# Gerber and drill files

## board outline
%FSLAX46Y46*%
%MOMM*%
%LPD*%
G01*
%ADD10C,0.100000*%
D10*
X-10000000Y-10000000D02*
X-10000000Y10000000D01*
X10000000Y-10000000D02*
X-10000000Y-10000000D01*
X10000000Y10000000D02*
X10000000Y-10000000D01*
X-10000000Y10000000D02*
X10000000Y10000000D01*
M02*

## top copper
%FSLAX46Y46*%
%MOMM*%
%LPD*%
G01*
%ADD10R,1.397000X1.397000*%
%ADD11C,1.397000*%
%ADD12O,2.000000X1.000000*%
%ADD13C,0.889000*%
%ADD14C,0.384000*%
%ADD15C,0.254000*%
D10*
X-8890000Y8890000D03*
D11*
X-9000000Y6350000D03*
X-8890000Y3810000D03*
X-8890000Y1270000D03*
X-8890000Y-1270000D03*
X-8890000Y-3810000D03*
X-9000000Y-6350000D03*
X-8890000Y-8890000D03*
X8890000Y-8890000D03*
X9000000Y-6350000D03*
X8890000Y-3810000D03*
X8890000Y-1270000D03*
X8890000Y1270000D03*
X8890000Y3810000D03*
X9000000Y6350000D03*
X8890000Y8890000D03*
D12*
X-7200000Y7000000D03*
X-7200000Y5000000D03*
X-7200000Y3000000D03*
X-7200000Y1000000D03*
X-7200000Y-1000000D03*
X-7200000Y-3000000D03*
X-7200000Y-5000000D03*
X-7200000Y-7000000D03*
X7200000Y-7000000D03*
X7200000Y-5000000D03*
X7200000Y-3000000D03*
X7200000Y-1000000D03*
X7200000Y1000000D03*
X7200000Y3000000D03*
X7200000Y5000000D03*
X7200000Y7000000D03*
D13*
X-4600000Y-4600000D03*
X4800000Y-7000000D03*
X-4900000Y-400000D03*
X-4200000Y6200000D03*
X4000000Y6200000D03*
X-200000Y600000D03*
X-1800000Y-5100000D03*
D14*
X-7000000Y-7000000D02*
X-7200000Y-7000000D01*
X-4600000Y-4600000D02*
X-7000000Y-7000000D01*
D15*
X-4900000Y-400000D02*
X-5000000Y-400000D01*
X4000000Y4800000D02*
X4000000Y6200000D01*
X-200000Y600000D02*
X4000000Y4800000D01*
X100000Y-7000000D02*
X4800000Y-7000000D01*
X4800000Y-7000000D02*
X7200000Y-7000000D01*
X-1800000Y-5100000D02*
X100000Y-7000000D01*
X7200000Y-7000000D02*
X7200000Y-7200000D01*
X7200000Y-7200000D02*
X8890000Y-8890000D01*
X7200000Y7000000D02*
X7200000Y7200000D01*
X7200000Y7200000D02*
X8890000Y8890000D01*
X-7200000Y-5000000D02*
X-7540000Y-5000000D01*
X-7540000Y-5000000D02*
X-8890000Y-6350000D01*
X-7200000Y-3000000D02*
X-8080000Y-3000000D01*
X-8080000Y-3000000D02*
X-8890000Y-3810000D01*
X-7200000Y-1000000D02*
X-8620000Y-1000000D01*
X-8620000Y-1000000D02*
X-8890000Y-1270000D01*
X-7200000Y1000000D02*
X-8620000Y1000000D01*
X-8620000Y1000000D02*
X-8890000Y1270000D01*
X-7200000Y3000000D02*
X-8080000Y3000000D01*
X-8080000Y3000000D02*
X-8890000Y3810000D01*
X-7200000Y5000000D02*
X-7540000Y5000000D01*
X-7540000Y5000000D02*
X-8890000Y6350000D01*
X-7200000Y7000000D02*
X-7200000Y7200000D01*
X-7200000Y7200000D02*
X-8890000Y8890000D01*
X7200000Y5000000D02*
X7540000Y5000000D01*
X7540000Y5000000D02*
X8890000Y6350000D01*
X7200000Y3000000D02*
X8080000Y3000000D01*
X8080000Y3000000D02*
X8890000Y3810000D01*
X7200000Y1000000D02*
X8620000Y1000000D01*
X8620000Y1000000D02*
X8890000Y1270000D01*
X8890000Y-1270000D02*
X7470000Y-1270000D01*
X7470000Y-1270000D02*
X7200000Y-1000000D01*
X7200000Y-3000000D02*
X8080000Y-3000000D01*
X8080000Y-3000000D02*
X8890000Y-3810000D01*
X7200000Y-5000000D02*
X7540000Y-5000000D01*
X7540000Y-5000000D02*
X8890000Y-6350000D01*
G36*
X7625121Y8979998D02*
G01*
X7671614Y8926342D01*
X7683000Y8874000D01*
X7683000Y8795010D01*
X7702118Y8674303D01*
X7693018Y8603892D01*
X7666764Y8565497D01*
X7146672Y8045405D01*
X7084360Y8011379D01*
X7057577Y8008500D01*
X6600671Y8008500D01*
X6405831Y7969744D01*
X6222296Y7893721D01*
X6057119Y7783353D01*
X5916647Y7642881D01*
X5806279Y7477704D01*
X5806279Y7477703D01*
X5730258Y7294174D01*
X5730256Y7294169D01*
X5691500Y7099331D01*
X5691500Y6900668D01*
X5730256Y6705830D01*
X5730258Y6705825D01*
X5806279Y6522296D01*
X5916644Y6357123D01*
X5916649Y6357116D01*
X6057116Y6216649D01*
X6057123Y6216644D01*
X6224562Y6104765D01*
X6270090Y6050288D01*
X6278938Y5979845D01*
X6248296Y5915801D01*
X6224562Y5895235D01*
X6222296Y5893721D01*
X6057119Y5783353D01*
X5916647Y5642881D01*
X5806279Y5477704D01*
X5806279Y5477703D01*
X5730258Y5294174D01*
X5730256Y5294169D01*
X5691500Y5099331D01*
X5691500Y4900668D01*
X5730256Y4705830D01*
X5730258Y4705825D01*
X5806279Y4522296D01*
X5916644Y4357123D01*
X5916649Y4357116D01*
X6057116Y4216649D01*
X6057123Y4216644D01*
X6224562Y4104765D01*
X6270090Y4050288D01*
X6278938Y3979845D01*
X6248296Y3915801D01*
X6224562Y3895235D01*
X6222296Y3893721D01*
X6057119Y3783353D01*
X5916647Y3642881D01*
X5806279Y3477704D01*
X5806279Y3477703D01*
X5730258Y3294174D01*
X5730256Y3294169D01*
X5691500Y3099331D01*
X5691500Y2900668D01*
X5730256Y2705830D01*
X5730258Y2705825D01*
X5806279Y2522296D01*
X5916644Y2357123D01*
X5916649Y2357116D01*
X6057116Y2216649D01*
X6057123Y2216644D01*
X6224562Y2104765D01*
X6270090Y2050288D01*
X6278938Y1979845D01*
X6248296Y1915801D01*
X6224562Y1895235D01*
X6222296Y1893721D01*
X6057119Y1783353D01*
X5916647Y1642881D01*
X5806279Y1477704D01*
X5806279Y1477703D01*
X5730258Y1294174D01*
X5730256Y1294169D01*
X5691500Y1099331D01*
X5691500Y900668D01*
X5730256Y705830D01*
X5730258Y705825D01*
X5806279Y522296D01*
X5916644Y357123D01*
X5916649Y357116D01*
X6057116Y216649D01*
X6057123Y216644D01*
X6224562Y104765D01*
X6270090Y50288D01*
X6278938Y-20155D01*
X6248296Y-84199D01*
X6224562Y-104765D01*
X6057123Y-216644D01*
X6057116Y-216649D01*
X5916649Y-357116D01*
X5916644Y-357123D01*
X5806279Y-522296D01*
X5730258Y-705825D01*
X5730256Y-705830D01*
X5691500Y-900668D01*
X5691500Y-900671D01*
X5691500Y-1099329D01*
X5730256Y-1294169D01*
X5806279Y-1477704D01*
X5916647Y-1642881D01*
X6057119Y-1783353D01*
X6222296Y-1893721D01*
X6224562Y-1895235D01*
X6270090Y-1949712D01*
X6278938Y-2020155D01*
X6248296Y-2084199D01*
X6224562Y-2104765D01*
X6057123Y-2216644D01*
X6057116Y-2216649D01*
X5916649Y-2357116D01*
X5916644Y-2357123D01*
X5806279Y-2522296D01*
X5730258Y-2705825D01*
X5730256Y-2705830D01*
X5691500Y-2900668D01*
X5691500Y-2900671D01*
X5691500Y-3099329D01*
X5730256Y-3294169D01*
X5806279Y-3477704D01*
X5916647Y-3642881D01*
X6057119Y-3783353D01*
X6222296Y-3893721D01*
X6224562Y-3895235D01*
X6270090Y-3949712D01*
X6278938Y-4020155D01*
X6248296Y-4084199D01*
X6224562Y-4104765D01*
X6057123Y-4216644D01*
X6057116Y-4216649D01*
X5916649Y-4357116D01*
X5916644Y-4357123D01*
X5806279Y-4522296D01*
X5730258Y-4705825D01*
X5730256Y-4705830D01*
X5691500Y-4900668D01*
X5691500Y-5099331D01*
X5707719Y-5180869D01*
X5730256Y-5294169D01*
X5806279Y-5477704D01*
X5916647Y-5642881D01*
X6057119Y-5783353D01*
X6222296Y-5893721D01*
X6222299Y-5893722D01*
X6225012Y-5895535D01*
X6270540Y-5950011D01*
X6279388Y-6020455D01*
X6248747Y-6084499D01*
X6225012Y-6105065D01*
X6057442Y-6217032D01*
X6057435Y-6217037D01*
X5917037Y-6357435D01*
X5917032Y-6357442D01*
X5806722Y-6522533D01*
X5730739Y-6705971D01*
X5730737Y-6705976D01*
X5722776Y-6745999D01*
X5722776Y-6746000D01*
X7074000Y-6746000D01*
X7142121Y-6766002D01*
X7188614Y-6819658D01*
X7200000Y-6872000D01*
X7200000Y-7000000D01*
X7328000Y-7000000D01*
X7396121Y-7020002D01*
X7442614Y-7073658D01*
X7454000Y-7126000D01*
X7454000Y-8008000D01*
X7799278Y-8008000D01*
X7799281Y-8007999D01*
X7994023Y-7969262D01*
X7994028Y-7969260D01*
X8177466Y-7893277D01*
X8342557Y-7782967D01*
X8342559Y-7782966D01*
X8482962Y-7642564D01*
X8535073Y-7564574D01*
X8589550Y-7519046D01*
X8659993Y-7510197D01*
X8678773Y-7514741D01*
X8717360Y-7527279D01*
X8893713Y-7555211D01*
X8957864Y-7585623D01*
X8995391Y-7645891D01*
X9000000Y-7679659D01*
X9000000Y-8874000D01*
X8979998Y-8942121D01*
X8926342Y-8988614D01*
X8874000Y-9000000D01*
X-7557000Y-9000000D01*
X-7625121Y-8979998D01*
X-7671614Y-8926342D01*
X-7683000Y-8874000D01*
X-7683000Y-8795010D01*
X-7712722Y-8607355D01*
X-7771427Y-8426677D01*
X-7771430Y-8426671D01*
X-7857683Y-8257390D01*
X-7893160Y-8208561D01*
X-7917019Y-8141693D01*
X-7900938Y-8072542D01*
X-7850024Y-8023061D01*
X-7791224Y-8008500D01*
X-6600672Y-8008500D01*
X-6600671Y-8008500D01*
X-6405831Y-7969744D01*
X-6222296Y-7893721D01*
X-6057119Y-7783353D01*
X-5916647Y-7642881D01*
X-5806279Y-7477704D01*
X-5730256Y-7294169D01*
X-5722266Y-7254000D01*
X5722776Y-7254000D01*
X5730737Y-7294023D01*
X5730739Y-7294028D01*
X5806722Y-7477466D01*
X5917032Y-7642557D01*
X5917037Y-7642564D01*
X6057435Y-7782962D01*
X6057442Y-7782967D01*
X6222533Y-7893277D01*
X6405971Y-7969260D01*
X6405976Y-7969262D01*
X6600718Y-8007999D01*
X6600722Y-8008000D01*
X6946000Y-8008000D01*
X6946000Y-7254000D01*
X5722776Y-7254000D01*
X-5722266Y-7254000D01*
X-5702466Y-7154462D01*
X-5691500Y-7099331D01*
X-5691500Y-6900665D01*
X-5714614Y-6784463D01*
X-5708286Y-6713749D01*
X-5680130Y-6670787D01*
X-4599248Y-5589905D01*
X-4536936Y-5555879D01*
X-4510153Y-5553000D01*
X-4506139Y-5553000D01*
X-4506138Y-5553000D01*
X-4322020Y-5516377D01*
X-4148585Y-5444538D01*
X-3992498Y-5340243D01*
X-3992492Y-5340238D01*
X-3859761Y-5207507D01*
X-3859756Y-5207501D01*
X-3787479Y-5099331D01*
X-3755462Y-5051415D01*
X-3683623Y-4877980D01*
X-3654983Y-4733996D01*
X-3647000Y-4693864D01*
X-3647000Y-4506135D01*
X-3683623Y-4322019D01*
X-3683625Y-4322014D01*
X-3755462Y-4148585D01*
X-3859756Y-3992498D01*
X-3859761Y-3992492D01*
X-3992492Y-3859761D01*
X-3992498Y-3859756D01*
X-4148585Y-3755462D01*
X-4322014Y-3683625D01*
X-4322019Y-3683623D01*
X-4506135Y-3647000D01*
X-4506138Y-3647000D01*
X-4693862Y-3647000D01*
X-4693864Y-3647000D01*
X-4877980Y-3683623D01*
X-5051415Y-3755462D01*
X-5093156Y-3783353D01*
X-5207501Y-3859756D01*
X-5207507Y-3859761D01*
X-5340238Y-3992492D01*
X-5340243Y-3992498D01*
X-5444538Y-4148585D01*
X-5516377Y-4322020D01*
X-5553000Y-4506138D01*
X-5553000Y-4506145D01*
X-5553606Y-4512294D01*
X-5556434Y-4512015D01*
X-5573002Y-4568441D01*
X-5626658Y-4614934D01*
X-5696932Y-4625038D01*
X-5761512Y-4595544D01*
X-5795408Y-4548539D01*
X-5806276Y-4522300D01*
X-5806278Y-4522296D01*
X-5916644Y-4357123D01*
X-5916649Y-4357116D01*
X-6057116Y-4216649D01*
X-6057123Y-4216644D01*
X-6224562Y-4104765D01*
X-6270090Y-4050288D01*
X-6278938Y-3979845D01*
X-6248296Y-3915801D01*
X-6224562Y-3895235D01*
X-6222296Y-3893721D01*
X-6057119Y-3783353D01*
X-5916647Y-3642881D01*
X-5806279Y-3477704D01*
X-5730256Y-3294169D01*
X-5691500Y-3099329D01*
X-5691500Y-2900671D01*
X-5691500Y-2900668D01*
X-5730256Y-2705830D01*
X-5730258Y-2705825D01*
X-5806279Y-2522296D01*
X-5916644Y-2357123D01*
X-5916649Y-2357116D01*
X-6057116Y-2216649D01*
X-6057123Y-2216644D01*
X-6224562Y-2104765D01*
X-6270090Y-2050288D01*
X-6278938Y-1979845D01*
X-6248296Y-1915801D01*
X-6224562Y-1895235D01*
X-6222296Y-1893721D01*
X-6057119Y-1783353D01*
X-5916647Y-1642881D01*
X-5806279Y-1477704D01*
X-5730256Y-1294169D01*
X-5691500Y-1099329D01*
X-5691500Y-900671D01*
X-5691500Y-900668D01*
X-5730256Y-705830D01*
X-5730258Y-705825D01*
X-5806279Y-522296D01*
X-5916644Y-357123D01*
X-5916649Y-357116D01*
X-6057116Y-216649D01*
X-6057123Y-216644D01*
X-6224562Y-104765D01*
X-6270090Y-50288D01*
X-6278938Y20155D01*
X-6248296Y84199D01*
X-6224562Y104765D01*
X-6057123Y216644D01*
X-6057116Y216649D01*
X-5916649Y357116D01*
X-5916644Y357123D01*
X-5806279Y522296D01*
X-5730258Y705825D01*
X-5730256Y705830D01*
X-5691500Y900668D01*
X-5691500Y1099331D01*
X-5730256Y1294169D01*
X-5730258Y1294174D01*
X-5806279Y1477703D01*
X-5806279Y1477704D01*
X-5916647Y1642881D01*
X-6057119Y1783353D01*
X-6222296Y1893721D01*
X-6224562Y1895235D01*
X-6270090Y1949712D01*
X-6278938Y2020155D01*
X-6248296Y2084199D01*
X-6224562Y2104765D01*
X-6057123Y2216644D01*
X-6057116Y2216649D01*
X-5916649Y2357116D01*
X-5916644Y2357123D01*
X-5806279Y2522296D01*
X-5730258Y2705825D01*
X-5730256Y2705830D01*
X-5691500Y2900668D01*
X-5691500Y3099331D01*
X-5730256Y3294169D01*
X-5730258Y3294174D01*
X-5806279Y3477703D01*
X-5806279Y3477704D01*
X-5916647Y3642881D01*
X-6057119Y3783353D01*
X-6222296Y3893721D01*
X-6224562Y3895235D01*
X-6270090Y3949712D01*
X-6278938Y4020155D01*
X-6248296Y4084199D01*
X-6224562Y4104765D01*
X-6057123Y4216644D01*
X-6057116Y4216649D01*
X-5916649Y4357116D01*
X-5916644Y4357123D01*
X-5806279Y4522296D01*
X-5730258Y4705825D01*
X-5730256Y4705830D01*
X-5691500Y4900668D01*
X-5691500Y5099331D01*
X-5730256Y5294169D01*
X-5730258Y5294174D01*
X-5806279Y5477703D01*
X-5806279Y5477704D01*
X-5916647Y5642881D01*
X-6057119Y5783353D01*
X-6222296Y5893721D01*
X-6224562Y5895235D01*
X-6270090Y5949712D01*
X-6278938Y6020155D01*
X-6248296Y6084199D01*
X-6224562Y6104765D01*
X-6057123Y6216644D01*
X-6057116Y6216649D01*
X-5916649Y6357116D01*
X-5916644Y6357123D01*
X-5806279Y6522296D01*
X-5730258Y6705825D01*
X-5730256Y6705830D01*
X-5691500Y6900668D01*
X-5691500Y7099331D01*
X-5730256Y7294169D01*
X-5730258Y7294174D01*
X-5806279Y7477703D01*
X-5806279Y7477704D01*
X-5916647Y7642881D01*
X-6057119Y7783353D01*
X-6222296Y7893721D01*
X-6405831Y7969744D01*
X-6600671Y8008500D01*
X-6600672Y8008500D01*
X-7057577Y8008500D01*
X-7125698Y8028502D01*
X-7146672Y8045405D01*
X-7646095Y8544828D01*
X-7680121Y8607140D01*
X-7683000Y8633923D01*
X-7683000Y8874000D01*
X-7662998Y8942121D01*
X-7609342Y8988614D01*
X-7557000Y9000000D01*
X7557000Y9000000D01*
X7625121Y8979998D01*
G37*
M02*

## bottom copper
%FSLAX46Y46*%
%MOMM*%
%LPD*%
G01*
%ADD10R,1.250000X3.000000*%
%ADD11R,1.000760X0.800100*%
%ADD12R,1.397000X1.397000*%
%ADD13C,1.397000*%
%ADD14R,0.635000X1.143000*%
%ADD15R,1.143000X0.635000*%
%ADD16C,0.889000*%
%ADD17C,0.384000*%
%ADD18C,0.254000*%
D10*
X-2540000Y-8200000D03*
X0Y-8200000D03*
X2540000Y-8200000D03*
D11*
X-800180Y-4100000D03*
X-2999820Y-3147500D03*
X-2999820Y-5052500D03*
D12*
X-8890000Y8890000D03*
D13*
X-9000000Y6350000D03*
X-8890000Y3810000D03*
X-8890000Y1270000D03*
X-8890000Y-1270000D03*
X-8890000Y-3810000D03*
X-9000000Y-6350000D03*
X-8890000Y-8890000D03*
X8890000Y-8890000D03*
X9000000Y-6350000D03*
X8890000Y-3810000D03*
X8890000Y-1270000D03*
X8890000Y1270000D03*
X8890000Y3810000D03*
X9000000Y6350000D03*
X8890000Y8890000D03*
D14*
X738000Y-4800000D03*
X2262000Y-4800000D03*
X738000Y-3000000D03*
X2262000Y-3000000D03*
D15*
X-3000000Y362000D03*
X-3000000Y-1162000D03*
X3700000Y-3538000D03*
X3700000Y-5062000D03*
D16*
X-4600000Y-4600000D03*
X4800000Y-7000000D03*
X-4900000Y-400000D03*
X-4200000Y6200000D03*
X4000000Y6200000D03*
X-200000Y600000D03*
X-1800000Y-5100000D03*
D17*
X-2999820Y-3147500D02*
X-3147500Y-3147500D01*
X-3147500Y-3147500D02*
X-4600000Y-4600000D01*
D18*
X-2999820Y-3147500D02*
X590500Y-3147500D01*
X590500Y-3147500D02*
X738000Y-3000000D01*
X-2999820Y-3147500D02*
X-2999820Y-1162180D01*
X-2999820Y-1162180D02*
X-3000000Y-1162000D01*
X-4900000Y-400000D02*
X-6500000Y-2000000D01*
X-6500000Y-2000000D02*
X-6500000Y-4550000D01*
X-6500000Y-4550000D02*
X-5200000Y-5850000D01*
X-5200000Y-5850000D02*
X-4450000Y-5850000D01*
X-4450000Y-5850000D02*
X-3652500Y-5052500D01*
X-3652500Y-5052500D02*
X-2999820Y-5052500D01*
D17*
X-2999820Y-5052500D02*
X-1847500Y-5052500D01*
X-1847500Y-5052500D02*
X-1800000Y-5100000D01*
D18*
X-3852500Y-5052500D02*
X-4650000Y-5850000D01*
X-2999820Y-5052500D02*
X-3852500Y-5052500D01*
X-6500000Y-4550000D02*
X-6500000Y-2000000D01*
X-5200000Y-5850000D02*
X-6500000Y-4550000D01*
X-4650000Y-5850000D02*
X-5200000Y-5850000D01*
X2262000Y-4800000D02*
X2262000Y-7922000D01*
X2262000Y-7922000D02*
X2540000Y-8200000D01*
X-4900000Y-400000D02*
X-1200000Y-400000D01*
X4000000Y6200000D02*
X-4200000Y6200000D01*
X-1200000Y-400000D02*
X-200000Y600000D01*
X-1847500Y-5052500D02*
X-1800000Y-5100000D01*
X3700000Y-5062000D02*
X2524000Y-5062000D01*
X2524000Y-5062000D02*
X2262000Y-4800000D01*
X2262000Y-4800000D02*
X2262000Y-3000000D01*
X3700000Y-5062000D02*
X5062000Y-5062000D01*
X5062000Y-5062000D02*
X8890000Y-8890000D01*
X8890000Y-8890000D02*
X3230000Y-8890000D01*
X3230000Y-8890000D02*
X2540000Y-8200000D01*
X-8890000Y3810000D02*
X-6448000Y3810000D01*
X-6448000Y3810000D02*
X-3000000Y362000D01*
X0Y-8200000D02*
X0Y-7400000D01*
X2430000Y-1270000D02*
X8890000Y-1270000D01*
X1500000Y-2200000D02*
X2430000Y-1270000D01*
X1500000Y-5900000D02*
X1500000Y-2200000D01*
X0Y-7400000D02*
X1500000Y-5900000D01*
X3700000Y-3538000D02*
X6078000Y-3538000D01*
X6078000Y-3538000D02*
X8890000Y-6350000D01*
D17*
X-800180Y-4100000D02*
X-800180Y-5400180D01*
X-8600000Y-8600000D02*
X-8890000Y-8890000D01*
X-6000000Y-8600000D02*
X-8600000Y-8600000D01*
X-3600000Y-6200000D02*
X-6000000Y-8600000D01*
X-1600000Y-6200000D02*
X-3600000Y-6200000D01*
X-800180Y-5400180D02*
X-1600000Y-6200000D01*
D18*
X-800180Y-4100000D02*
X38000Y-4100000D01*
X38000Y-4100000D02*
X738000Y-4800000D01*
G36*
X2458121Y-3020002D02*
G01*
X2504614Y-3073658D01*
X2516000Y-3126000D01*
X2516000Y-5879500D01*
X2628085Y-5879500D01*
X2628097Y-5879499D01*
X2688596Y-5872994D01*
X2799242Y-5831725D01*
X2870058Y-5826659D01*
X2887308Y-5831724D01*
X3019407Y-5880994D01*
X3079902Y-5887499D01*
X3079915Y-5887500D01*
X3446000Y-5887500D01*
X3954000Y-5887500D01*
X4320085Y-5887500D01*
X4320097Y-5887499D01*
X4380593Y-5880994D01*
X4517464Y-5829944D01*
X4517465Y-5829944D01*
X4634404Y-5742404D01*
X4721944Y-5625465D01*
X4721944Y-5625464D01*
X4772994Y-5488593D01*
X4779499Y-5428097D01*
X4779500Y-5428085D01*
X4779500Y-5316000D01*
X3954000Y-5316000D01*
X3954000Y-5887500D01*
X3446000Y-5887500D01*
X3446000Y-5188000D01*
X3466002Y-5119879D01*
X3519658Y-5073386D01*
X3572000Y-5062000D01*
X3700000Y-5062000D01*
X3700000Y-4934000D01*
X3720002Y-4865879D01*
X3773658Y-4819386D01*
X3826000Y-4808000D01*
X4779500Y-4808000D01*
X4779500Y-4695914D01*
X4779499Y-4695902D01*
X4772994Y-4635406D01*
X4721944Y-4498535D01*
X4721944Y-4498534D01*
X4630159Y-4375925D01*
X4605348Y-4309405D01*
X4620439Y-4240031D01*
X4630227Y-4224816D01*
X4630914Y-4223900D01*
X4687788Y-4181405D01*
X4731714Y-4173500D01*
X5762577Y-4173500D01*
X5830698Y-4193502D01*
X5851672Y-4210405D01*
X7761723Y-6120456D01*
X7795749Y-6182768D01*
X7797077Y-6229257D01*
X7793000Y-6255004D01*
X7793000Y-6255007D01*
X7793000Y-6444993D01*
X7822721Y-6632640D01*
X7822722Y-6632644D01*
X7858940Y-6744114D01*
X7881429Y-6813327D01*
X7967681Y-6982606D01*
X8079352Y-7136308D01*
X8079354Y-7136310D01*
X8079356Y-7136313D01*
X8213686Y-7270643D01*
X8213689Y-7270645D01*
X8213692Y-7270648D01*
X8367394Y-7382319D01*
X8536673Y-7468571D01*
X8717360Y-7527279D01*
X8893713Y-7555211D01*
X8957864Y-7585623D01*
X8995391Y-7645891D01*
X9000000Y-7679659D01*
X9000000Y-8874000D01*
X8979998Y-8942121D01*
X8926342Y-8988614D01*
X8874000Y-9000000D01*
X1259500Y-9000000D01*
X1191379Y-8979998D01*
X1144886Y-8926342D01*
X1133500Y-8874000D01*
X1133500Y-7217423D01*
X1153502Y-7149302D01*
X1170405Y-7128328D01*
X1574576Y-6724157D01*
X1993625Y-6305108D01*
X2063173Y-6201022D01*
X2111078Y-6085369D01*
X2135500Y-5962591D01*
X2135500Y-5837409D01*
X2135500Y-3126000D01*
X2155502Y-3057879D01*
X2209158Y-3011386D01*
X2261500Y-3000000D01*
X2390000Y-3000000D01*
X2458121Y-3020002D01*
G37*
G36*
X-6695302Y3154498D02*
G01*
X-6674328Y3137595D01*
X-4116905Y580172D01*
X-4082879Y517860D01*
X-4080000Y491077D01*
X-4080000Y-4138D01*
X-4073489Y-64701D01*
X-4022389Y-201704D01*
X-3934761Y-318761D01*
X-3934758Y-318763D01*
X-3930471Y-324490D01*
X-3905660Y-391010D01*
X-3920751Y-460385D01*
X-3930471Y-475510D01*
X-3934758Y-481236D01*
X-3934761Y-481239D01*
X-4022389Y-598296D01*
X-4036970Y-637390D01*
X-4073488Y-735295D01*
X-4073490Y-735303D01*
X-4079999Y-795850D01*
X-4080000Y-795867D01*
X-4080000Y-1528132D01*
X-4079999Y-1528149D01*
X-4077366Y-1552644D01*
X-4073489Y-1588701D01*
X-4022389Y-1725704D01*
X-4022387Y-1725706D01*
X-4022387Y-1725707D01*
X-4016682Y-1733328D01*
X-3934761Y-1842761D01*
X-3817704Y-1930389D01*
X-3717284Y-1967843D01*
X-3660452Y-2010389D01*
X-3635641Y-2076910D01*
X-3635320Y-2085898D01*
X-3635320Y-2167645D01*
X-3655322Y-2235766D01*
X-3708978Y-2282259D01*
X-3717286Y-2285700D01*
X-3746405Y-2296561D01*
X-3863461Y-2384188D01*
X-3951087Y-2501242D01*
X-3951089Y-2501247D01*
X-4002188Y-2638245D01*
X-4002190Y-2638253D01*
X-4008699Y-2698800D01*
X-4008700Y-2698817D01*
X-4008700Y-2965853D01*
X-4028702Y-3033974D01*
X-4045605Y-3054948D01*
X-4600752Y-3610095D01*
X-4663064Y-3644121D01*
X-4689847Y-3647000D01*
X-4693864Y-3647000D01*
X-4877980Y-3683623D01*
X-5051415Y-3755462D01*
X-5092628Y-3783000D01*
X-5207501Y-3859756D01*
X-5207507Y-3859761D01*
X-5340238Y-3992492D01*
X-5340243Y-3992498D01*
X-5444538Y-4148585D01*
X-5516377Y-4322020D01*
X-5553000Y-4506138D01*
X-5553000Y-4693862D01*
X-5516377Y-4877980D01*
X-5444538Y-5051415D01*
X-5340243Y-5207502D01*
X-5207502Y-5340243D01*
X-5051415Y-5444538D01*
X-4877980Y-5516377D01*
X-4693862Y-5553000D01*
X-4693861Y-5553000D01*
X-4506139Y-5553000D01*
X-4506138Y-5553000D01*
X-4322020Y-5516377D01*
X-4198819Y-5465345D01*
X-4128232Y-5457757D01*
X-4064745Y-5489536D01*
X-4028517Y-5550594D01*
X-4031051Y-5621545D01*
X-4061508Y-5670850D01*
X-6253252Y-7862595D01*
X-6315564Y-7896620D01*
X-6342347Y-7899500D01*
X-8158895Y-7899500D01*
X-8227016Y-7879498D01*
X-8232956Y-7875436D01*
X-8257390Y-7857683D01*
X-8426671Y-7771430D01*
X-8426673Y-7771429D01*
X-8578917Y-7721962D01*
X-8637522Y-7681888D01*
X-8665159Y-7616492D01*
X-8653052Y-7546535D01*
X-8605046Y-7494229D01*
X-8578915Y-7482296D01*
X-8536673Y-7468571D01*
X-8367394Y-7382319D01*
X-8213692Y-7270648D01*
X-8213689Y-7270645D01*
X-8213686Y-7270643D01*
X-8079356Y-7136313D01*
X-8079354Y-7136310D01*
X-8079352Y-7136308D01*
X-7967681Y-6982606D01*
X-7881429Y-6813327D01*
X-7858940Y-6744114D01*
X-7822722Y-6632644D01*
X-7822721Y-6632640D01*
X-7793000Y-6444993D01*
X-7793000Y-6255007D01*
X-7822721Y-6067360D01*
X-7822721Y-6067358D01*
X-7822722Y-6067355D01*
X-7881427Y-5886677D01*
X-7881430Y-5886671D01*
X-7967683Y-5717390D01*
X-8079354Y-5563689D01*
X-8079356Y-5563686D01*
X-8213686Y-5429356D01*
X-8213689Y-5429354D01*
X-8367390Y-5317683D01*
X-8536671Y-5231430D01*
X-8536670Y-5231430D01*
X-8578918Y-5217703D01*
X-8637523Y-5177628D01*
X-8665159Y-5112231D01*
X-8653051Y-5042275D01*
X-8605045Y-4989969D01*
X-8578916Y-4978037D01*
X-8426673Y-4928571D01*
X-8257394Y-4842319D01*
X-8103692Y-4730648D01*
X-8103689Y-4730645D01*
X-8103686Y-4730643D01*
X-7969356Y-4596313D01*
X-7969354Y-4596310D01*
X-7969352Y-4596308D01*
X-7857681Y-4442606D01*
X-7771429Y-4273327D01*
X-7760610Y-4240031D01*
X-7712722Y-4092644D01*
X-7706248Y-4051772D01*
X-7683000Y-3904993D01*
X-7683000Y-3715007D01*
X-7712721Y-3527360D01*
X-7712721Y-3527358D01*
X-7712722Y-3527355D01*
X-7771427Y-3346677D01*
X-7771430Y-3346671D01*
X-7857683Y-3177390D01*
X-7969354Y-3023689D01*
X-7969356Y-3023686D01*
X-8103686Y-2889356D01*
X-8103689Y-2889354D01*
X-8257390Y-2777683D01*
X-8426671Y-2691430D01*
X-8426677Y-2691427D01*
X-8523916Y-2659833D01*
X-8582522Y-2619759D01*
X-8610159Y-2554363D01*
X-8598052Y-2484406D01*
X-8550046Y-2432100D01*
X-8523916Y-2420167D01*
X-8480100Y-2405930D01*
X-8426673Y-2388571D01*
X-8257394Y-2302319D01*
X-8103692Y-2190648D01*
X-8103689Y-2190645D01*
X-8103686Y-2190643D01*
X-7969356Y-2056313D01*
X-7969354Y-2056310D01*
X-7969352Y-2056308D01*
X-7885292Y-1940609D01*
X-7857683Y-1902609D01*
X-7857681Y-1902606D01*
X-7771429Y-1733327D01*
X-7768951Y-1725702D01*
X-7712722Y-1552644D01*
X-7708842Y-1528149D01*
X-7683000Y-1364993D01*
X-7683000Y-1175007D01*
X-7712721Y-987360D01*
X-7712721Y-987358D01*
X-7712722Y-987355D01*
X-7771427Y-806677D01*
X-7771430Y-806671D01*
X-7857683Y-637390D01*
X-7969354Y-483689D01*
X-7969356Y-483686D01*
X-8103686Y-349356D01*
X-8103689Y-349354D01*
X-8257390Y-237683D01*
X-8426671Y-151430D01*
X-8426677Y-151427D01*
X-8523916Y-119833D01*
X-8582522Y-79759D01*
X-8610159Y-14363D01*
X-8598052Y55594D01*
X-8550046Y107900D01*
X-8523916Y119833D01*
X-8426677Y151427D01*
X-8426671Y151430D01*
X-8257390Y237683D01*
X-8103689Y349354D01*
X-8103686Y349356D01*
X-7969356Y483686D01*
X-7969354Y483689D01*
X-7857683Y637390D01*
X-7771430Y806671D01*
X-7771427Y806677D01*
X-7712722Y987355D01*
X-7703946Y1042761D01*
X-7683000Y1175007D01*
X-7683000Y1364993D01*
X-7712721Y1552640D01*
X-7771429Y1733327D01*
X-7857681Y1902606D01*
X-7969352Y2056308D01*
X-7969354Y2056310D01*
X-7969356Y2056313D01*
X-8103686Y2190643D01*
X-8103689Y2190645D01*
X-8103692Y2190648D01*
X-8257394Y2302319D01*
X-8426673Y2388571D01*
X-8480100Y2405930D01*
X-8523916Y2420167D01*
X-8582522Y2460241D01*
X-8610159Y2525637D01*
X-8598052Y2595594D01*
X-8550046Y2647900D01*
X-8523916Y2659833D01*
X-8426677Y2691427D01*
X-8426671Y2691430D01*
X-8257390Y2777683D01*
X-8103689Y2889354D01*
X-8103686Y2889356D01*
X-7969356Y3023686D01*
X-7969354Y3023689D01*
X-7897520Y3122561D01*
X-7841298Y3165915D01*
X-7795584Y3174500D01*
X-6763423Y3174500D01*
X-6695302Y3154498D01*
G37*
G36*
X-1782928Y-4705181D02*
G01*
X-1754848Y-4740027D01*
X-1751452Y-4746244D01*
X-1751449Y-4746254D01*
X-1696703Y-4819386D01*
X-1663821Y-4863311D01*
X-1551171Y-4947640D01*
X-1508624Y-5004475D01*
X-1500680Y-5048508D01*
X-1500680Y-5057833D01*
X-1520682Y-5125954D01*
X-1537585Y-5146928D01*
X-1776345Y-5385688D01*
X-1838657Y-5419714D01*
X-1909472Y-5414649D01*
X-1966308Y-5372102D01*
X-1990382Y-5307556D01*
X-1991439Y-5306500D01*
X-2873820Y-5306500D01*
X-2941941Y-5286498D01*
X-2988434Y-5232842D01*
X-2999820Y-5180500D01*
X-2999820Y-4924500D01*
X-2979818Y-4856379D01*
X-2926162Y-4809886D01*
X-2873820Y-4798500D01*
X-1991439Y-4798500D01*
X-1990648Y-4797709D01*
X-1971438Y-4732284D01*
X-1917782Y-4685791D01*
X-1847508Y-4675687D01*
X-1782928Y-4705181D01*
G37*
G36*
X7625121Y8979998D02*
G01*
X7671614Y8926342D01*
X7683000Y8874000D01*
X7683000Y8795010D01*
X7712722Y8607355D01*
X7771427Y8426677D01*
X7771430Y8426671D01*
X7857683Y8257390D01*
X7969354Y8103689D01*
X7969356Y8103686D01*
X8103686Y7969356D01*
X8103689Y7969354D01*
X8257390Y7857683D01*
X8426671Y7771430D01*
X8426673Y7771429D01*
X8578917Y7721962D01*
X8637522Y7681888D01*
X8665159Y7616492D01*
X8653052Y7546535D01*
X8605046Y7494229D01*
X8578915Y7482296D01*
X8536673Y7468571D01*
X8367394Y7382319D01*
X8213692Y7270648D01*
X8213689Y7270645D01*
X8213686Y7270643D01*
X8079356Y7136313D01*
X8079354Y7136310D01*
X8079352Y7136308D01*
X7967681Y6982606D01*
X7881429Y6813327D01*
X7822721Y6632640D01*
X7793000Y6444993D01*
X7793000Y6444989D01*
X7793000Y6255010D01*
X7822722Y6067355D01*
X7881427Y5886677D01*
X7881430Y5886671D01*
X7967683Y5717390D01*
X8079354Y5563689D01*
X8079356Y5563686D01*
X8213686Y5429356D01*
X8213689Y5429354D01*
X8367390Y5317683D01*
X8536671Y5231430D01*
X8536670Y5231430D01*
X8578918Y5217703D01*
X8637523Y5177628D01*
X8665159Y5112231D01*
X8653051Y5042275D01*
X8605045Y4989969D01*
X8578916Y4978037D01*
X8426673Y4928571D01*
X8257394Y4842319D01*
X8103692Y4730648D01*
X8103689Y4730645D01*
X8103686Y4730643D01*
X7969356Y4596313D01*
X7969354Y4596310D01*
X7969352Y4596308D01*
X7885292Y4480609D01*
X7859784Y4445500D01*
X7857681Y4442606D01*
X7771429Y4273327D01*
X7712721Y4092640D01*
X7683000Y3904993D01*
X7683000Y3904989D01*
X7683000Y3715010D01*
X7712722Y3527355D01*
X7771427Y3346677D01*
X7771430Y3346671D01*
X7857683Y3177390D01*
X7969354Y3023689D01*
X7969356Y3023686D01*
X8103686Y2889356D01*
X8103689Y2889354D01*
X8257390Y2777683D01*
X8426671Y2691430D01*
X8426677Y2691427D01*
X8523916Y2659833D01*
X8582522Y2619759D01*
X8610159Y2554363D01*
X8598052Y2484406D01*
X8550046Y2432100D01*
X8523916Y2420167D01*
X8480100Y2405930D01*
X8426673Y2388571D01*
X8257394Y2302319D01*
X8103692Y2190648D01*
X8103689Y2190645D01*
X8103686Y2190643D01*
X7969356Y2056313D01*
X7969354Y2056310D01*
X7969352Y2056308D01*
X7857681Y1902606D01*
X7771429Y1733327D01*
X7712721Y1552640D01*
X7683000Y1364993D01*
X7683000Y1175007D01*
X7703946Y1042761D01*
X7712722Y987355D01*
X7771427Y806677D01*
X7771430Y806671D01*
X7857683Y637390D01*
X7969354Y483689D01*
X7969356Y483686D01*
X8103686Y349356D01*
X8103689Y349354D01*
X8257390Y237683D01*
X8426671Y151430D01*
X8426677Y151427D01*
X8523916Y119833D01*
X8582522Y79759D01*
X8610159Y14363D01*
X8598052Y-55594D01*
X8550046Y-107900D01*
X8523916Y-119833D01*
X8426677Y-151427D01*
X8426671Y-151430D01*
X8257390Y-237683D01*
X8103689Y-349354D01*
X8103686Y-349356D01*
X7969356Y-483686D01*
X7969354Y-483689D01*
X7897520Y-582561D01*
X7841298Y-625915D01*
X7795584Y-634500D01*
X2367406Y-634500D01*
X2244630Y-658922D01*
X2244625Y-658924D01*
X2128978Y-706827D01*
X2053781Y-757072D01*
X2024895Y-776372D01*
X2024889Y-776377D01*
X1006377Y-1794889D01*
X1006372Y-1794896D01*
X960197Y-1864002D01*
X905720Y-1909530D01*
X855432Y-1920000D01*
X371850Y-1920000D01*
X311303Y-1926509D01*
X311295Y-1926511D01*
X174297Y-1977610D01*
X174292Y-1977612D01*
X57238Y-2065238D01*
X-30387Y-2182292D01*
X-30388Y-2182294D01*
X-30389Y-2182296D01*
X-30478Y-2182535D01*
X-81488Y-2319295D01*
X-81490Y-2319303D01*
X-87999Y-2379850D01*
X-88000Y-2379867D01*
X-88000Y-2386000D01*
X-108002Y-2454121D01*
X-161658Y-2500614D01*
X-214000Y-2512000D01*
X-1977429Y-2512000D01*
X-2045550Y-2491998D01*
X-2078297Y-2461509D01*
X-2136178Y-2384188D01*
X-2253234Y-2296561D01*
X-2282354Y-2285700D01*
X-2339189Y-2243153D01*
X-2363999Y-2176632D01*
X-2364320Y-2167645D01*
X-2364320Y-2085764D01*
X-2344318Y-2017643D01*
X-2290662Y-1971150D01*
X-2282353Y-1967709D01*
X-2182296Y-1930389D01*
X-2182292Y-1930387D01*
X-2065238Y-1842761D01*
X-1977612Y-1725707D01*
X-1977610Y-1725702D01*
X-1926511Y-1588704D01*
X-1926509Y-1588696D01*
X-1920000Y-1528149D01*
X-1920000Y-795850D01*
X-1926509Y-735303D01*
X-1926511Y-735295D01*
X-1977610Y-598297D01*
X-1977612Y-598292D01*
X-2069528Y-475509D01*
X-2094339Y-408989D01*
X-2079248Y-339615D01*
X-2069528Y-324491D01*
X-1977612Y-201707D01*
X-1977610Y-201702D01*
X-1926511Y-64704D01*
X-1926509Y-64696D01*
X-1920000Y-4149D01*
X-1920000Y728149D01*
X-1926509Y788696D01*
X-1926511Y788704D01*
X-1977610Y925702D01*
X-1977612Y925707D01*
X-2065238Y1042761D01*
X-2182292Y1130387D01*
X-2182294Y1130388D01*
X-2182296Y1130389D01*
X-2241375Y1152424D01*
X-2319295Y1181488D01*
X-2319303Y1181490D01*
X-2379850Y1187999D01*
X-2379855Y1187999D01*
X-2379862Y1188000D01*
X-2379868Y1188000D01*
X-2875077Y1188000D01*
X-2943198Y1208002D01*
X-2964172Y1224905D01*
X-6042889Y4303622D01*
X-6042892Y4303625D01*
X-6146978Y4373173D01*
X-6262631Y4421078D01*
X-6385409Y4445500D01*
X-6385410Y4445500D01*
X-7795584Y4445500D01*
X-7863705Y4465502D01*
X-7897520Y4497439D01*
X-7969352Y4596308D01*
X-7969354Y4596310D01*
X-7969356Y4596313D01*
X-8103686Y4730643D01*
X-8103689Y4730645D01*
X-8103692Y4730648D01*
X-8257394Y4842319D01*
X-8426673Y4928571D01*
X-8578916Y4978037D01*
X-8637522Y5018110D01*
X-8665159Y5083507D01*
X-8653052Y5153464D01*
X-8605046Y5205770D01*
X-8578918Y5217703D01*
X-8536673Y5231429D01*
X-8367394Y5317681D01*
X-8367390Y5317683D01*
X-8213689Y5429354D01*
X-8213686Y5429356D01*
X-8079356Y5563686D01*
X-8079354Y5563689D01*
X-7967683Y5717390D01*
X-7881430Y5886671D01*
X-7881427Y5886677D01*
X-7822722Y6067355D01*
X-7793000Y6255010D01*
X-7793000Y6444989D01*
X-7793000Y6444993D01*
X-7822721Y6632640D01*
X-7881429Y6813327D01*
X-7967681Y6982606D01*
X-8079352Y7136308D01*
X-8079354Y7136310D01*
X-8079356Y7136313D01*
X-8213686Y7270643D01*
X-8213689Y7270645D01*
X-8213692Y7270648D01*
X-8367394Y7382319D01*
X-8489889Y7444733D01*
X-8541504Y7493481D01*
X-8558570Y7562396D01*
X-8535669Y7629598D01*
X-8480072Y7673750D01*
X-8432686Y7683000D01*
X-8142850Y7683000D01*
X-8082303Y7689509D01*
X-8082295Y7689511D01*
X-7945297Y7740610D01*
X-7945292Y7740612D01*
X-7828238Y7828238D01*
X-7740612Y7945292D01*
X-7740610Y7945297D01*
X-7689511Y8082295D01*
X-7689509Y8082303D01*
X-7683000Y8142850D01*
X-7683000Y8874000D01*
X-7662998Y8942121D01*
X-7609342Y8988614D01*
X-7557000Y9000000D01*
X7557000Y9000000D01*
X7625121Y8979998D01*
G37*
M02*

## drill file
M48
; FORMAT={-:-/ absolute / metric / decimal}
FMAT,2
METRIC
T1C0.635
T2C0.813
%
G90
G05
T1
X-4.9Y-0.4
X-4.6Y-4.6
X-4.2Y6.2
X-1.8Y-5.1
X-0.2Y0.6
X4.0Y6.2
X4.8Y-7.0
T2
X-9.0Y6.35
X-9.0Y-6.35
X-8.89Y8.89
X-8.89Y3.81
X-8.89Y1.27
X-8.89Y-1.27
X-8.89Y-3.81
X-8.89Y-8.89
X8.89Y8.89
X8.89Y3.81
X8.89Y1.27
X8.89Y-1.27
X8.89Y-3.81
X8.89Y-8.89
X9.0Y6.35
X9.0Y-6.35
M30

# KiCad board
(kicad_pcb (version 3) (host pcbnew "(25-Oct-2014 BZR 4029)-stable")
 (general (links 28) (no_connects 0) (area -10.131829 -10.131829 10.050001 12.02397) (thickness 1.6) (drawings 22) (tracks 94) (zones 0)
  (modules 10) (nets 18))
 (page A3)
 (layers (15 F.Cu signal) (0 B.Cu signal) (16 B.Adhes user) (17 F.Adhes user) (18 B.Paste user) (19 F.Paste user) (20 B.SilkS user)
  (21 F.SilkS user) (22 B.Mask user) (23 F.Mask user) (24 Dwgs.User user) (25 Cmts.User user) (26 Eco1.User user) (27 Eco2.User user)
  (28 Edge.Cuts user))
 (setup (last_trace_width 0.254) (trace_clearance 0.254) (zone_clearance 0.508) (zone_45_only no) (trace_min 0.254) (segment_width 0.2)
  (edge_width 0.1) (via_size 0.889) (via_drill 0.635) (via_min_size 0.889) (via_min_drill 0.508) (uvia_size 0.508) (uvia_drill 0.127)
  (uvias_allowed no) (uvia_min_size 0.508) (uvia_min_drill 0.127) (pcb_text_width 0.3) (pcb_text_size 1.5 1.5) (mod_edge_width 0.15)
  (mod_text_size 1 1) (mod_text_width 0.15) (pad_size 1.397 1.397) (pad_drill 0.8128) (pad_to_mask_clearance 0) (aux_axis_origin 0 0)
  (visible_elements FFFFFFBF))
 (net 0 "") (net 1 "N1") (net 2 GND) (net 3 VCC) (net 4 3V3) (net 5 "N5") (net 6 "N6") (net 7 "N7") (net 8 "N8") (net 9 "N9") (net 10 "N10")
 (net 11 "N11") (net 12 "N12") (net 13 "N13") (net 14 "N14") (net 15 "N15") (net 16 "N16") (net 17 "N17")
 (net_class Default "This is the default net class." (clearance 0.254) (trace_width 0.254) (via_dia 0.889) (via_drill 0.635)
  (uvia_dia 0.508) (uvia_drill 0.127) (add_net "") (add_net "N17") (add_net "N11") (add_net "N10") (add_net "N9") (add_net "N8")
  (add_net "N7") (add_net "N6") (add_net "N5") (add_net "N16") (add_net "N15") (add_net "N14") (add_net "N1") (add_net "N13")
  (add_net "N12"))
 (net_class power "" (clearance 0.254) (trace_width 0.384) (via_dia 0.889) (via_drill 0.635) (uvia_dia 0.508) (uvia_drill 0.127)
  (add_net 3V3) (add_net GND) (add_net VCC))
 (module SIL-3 (layer B.Cu) (at 0 8.2)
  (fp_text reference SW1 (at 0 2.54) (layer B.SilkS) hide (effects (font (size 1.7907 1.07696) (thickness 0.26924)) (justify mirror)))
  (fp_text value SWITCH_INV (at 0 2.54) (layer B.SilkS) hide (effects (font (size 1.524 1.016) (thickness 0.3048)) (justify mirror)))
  (pad 1 smd rect (at -2.54 0) (size 1.25 3) (layers B.Cu B.Paste B.Mask))
  (pad 2 smd rect (at 0 0) (size 1.25 3) (layers B.Cu B.Paste B.Mask) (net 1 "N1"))
  (pad 3 smd rect (at 2.54 0) (size 1.25 3) (layers B.Cu B.Paste B.Mask) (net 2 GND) (zone_connect 2)))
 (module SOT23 (layer B.Cu) (at -1.9 4.1 90)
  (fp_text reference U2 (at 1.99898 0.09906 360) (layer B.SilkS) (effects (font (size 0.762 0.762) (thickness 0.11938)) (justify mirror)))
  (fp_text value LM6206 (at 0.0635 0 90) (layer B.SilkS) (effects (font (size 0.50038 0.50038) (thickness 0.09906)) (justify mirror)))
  (pad 3 smd rect (at 0 1.09982 90) (size 0.8001 1.00076) (layers B.Cu B.Paste B.Mask) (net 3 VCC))
  (pad 2 smd rect (at 0.9525 -1.09982 90) (size 0.8001 1.00076) (layers B.Cu B.Paste B.Mask) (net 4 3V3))
  (pad 1 smd rect (at -0.9525 -1.09982 90) (size 0.8001 1.00076) (layers B.Cu B.Paste B.Mask) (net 2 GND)))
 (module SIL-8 (layer F.Cu) (at -8.89 0 270)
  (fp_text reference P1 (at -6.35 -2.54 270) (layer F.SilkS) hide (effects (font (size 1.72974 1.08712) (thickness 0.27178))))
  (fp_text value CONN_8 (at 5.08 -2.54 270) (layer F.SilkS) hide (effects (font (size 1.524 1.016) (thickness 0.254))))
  (pad 1 thru_hole rect (at -8.89 0 270) (size 1.397 1.397) (drill 0.8128) (layers *.Cu *.Mask F.SilkS) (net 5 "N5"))
  (pad 2 thru_hole circle (at -6.35 0.11 270) (size 1.397 1.397) (drill 0.8128) (layers *.Cu *.Mask F.SilkS) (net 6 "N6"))
  (pad 3 thru_hole circle (at -3.81 0 270) (size 1.397 1.397) (drill 0.8128) (layers *.Cu *.Mask F.SilkS) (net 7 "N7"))
  (pad 4 thru_hole circle (at -1.27 0 270) (size 1.397 1.397) (drill 0.8128) (layers *.Cu *.Mask F.SilkS) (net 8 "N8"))
  (pad 5 thru_hole circle (at 1.27 0 270) (size 1.397 1.397) (drill 0.8128) (layers *.Cu *.Mask F.SilkS) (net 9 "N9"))
  (pad 6 thru_hole circle (at 3.81 0 270) (size 1.397 1.397) (drill 0.8128) (layers *.Cu *.Mask F.SilkS) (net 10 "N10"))
  (pad 7 thru_hole circle (at 6.35 0.11 270) (size 1.397 1.397) (drill 0.8128) (layers *.Cu *.Mask F.SilkS) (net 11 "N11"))
  (pad 8 thru_hole circle (at 8.89 0 270) (size 1.397 1.397) (drill 0.8128) (layers *.Cu *.Mask F.SilkS) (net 3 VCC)))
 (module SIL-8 (layer F.Cu) (at 8.89 0 90)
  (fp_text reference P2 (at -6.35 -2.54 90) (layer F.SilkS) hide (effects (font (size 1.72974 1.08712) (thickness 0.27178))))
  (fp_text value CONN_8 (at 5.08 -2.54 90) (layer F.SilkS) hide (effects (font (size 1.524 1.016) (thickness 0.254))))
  (pad 1 thru_hole circle (at -8.89 0 90) (size 1.397 1.397) (drill 0.8128) (layers *.Cu *.Mask F.SilkS) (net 2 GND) (zone_connect 2))
  (pad 2 thru_hole circle (at -6.35 0.11 90) (size 1.397 1.397) (drill 0.8128) (layers *.Cu *.Mask F.SilkS) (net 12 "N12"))
  (pad 3 thru_hole circle (at -3.81 0 90) (size 1.397 1.397) (drill 0.8128) (layers *.Cu *.Mask F.SilkS) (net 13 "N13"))
  (pad 4 thru_hole circle (at -1.27 0 90) (size 1.397 1.397) (drill 0.8128) (layers *.Cu *.Mask F.SilkS) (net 1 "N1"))
  (pad 5 thru_hole circle (at 1.27 0 90) (size 1.397 1.397) (drill 0.8128) (layers *.Cu *.Mask F.SilkS) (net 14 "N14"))
  (pad 6 thru_hole circle (at 3.81 0 90) (size 1.397 1.397) (drill 0.8128) (layers *.Cu *.Mask F.SilkS) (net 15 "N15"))
  (pad 7 thru_hole circle (at 6.35 0.11 90) (size 1.397 1.397) (drill 0.8128) (layers *.Cu *.Mask F.SilkS) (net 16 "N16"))
  (pad 8 thru_hole circle (at 8.89 0 90) (size 1.397 1.397) (drill 0.8128) (layers *.Cu *.Mask F.SilkS) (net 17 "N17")))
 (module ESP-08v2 (layer F.Cu) (at 0 0)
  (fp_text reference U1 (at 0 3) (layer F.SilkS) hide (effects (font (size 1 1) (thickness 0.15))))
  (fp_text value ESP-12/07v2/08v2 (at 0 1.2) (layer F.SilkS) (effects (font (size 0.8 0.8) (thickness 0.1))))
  (pad 1 smd oval (at -7.2 -7) (size 2 1) (layers F.Cu F.Paste F.Mask) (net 5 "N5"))
  (pad 2 smd oval (at -7.2 -5) (size 2 1) (layers F.Cu F.Paste F.Mask) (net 6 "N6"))
  (pad 3 smd oval (at -7.2 -3) (size 2 1) (layers F.Cu F.Paste F.Mask) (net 7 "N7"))
  (pad 4 smd oval (at -7.2 -1) (size 2 1) (layers F.Cu F.Paste F.Mask) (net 8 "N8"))
  (pad 5 smd oval (at -7.2 1) (size 2 1) (layers F.Cu F.Paste F.Mask) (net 9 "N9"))
  (pad 6 smd oval (at -7.2 3) (size 2 1) (layers F.Cu F.Paste F.Mask) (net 10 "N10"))
  (pad 7 smd oval (at -7.2 5) (size 2 1) (layers F.Cu F.Paste F.Mask) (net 11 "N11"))
  (pad 8 smd oval (at -7.2 7) (size 2 1) (layers F.Cu F.Paste F.Mask) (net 4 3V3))
  (pad 9 smd oval (at 7.2 7) (size 2 1) (layers F.Cu F.Paste F.Mask) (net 2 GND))
  (pad 10 smd oval (at 7.2 5) (size 2 1) (layers F.Cu F.Paste F.Mask) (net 12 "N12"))
  (pad 11 smd oval (at 7.2 3) (size 2 1) (layers F.Cu F.Paste F.Mask) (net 13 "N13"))
  (pad 12 smd oval (at 7.2 1) (size 2 1) (layers F.Cu F.Paste F.Mask) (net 1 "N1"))
  (pad 13 smd oval (at 7.2 -1) (size 2 1) (layers F.Cu F.Paste F.Mask) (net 14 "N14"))
  (pad 14 smd oval (at 7.2 -3) (size 2 1) (layers F.Cu F.Paste F.Mask) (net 15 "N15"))
  (pad 15 smd oval (at 7.2 -5) (size 2 1) (layers F.Cu F.Paste F.Mask) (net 16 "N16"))
  (pad 16 smd oval (at 7.2 -7) (size 2 1) (layers F.Cu F.Paste F.Mask) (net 17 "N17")))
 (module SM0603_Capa (layer B.Cu) (at 1.5 4.8)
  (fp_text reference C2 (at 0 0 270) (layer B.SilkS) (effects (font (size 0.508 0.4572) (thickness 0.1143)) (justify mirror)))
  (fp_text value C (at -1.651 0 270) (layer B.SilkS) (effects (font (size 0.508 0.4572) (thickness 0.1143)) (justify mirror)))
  (pad 1 smd rect (at -0.762 0) (size 0.635 1.143) (layers B.Cu B.Paste B.Mask) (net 3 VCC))
  (pad 2 smd rect (at 0.762 0) (size 0.635 1.143) (layers B.Cu B.Paste B.Mask) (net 2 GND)))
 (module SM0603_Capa (layer B.Cu) (at 1.5 3)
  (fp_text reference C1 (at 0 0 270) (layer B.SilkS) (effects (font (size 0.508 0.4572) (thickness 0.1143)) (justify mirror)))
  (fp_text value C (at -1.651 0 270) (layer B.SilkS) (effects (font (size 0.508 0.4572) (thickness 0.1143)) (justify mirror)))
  (pad 1 smd rect (at -0.762 0) (size 0.635 1.143) (layers B.Cu B.Paste B.Mask) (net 4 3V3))
  (pad 2 smd rect (at 0.762 0) (size 0.635 1.143) (layers B.Cu B.Paste B.Mask) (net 2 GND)))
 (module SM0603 (layer B.Cu) (at -3 0.4 270)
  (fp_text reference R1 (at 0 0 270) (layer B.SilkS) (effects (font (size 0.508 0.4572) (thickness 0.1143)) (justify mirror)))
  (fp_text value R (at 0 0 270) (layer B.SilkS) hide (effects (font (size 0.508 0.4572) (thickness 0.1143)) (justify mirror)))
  (pad 1 smd rect (at -0.762 0 270) (size 0.635 1.143) (layers B.Cu B.Paste B.Mask) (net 7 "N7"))
  (pad 2 smd rect (at 0.762 0 270) (size 0.635 1.143) (layers B.Cu B.Paste B.Mask) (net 4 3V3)))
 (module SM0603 (layer B.Cu) (at 3.7 4.3 270)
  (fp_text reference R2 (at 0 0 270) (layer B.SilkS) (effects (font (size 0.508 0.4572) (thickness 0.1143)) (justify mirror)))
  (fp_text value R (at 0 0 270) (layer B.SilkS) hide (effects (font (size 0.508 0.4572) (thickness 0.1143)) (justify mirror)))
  (pad 1 smd rect (at -0.762 0 270) (size 0.635 1.143) (layers B.Cu B.Paste B.Mask) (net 12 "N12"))
  (pad 2 smd rect (at 0.762 0 270) (size 0.635 1.143) (layers B.Cu B.Paste B.Mask) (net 2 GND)))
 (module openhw (layer B.Cu) (at 0 -3.8)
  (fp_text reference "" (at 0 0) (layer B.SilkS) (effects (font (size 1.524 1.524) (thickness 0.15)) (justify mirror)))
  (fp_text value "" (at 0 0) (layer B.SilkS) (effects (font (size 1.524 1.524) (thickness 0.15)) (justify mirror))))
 (gr_line (start -10 10) (end -10 -10) (angle 90) (layer Edge.Cuts) (width 0.1))
 (gr_line (start 10 10) (end -10 10) (angle 90) (layer Edge.Cuts) (width 0.1))
 (gr_line (start 10 -10) (end 10 10) (angle 90) (layer Edge.Cuts) (width 0.1))
 (gr_line (start -10 -10) (end 10 -10) (angle 90) (layer Edge.Cuts) (width 0.1))
 (segment (start -2.99982 3.1475) (end -3.1475 3.1475) (width 0.384) (layer B.Cu) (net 4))
 (segment (start -7 7) (end -7.2 7) (width 0.384) (layer F.Cu) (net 4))
 (segment (start -4.6 4.6) (end -7 7) (width 0.384) (layer F.Cu) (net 4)) (via (at -4.6 4.6) (size 0.889) (layers F.Cu B.Cu) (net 4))
 (segment (start -3.1475 3.1475) (end -4.6 4.6) (width 0.384) (layer B.Cu) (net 4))
 (segment (start -2.99982 3.1475) (end 0.5905 3.1475) (width 0.254) (layer B.Cu) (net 4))
 (segment (start 0.5905 3.1475) (end 0.738 3) (width 0.254) (layer B.Cu) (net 4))
 (segment (start -2.99982 3.1475) (end -2.99982 1.16218) (width 0.254) (layer B.Cu) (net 4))
 (segment (start -2.99982 1.16218) (end -3 1.162) (width 0.254) (layer B.Cu) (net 4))
 (segment (start -4.9 0.4) (end -6.5 2) (width 0.254) (layer B.Cu) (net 2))
 (segment (start -6.5 2) (end -6.5 4.55) (width 0.254) (layer B.Cu) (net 2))
 (segment (start -6.5 4.55) (end -5.2 5.85) (width 0.254) (layer B.Cu) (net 2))
 (segment (start -5.2 5.85) (end -4.45 5.85) (width 0.254) (layer B.Cu) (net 2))
 (segment (start -4.45 5.85) (end -3.6525 5.0525) (width 0.254) (layer B.Cu) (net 2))
 (segment (start -3.6525 5.0525) (end -2.99982 5.0525) (width 0.254) (layer B.Cu) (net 2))
 (segment (start -2.99982 5.0525) (end -1.8475 5.0525) (width 0.384) (layer B.Cu) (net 2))
 (segment (start -1.8475 5.0525) (end -1.8 5.1) (width 0.384) (layer B.Cu) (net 2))
 (segment (start -3.8525 5.0525) (end -4.65 5.85) (width 0.254) (layer B.Cu) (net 2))
 (segment (start -2.99982 5.0525) (end -3.8525 5.0525) (width 0.254) (layer B.Cu) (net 2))
 (segment (start -6.5 4.55) (end -6.5 2) (width 0.254) (layer B.Cu) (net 2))
 (segment (start -5.2 5.85) (end -6.5 4.55) (width 0.254) (layer B.Cu) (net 2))
 (segment (start -4.65 5.85) (end -5.2 5.85) (width 0.254) (layer B.Cu) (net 2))
 (segment (start 2.262 4.8) (end 2.262 7.922) (width 0.254) (layer B.Cu) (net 2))
 (segment (start 2.262 7.922) (end 2.54 8.2) (width 0.254) (layer B.Cu) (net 2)) (via (at 4.8 7) (size 0.889) (layers F.Cu B.Cu) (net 2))
 (via (at -4.9 0.4) (size 0.889) (layers F.Cu B.Cu) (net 2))
 (segment (start -4.9 0.4) (end -5 0.4) (width 0.254) (layer F.Cu) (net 2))
 (segment (start -4.9 0.4) (end -1.2 0.4) (width 0.254) (layer B.Cu) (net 2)) (via (at -4.2 -6.2) (size 0.889) (layers F.Cu B.Cu) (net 2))
 (segment (start 4 -6.2) (end -4.2 -6.2) (width 0.254) (layer B.Cu) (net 2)) (via (at 4 -6.2) (size 0.889) (layers F.Cu B.Cu) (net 2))
 (segment (start 4 -4.8) (end 4 -6.2) (width 0.254) (layer F.Cu) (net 2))
 (segment (start -0.2 -0.6) (end 4 -4.8) (width 0.254) (layer F.Cu) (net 2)) (via (at -0.2 -0.6) (size 0.889) (layers F.Cu B.Cu) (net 2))
 (segment (start -1.2 0.4) (end -0.2 -0.6) (width 0.254) (layer B.Cu) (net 2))
 (segment (start 0.1 7) (end 4.8 7) (width 0.254) (layer F.Cu) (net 2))
 (segment (start 4.8 7) (end 7.2 7) (width 0.254) (layer F.Cu) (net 2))
 (segment (start -1.8 5.1) (end 0.1 7) (width 0.254) (layer F.Cu) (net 2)) (via (at -1.8 5.1) (size 0.889) (layers F.Cu B.Cu) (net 2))
 (segment (start -1.8475 5.0525) (end -1.8 5.1) (width 0.254) (layer B.Cu) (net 2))
 (segment (start 3.7 5.062) (end 2.524 5.062) (width 0.254) (layer B.Cu) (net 2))
 (segment (start 2.524 5.062) (end 2.262 4.8) (width 0.254) (layer B.Cu) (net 2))
 (segment (start 2.262 4.8) (end 2.262 3) (width 0.254) (layer B.Cu) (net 2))
 (segment (start 3.7 5.062) (end 5.062 5.062) (width 0.254) (layer B.Cu) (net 2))
 (segment (start 5.062 5.062) (end 8.89 8.89) (width 0.254) (layer B.Cu) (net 2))
 (segment (start 8.89 8.89) (end 3.23 8.89) (width 0.254) (layer B.Cu) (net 2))
 (segment (start 3.23 8.89) (end 2.54 8.2) (width 0.254) (layer B.Cu) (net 2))
 (segment (start 7.2 7) (end 7.2 7.2) (width 0.254) (layer F.Cu) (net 2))
 (segment (start 7.2 7.2) (end 8.89 8.89) (width 0.254) (layer F.Cu) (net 2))
 (segment (start 7.2 -7) (end 7.2 -7.2) (width 0.254) (layer F.Cu) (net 17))
 (segment (start 7.2 -7.2) (end 8.89 -8.89) (width 0.254) (layer F.Cu) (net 17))
 (segment (start -7.2 5) (end -7.54 5) (width 0.254) (layer F.Cu) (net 11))
 (segment (start -7.54 5) (end -8.89 6.35) (width 0.254) (layer F.Cu) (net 11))
 (segment (start -7.2 3) (end -8.08 3) (width 0.254) (layer F.Cu) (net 10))
 (segment (start -8.08 3) (end -8.89 3.81) (width 0.254) (layer F.Cu) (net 10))
 (segment (start -7.2 1) (end -8.62 1) (width 0.254) (layer F.Cu) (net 9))
 (segment (start -8.62 1) (end -8.89 1.27) (width 0.254) (layer F.Cu) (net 9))
 (segment (start -7.2 -1) (end -8.62 -1) (width 0.254) (layer F.Cu) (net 8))
 (segment (start -8.62 -1) (end -8.89 -1.27) (width 0.254) (layer F.Cu) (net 8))
 (segment (start -8.89 -3.81) (end -6.448 -3.81) (width 0.254) (layer B.Cu) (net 7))
 (segment (start -6.448 -3.81) (end -3 -0.362) (width 0.254) (layer B.Cu) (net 7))
 (segment (start -7.2 -3) (end -8.08 -3) (width 0.254) (layer F.Cu) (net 7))
 (segment (start -8.08 -3) (end -8.89 -3.81) (width 0.254) (layer F.Cu) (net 7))
 (segment (start -7.2 -5) (end -7.54 -5) (width 0.254) (layer F.Cu) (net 6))
 (segment (start -7.54 -5) (end -8.89 -6.35) (width 0.254) (layer F.Cu) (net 6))
 (segment (start -7.2 -7) (end -7.2 -7.2) (width 0.254) (layer F.Cu) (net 5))
 (segment (start -7.2 -7.2) (end -8.89 -8.89) (width 0.254) (layer F.Cu) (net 5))
 (segment (start 7.2 -5) (end 7.54 -5) (width 0.254) (layer F.Cu) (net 16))
 (segment (start 7.54 -5) (end 8.89 -6.35) (width 0.254) (layer F.Cu) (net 16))
 (segment (start 7.2 -3) (end 8.08 -3) (width 0.254) (layer F.Cu) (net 15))
 (segment (start 8.08 -3) (end 8.89 -3.81) (width 0.254) (layer F.Cu) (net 15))
 (segment (start 7.2 -1) (end 8.62 -1) (width 0.254) (layer F.Cu) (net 14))
 (segment (start 8.62 -1) (end 8.89 -1.27) (width 0.254) (layer F.Cu) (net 14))
 (segment (start 8.89 1.27) (end 7.47 1.27) (width 0.254) (layer F.Cu) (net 1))
 (segment (start 7.47 1.27) (end 7.2 1) (width 0.254) (layer F.Cu) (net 1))
 (segment (start 0 8.2) (end 0 7.4) (width 0.254) (layer B.Cu) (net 1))
 (segment (start 2.43 1.27) (end 8.89 1.27) (width 0.254) (layer B.Cu) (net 1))
 (segment (start 1.5 2.2) (end 2.43 1.27) (width 0.254) (layer B.Cu) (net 1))
 (segment (start 1.5 5.9) (end 1.5 2.2) (width 0.254) (layer B.Cu) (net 1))
 (segment (start 0 7.4) (end 1.5 5.9) (width 0.254) (layer B.Cu) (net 1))
 (segment (start 7.2 3) (end 8.08 3) (width 0.254) (layer F.Cu) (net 13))
 (segment (start 8.08 3) (end 8.89 3.81) (width 0.254) (layer F.Cu) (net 13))
 (segment (start 3.7 3.538) (end 6.078 3.538) (width 0.254) (layer B.Cu) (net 12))
 (segment (start 6.078 3.538) (end 8.89 6.35) (width 0.254) (layer B.Cu) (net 12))
 (segment (start 7.2 5) (end 7.54 5) (width 0.254) (layer F.Cu) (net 12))
 (segment (start 7.54 5) (end 8.89 6.35) (width 0.254) (layer F.Cu) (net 12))
 (segment (start -0.80018 4.1) (end -0.80018 5.40018) (width 0.384) (layer B.Cu) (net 3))
 (segment (start -8.6 8.6) (end -8.89 8.89) (width 0.384) (layer B.Cu) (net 3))
 (segment (start -6 8.6) (end -8.6 8.6) (width 0.384) (layer B.Cu) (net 3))
 (segment (start -3.6 6.2) (end -6 8.6) (width 0.384) (layer B.Cu) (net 3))
 (segment (start -1.6 6.2) (end -3.6 6.2) (width 0.384) (layer B.Cu) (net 3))
 (segment (start -0.80018 5.40018) (end -1.6 6.2) (width 0.384) (layer B.Cu) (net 3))
 (segment (start -0.80018 4.1) (end 0.038 4.1) (width 0.254) (layer B.Cu) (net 3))
 (segment (start 0.038 4.1) (end 0.738 4.8) (width 0.254) (layer B.Cu) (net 3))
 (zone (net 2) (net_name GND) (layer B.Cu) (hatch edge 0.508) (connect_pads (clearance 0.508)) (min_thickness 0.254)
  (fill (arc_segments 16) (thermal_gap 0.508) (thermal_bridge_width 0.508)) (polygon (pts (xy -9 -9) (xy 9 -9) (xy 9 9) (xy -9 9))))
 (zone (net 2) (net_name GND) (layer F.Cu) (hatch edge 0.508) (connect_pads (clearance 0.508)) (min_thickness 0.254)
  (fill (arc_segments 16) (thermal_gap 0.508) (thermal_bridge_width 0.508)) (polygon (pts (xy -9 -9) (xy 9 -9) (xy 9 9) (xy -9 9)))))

